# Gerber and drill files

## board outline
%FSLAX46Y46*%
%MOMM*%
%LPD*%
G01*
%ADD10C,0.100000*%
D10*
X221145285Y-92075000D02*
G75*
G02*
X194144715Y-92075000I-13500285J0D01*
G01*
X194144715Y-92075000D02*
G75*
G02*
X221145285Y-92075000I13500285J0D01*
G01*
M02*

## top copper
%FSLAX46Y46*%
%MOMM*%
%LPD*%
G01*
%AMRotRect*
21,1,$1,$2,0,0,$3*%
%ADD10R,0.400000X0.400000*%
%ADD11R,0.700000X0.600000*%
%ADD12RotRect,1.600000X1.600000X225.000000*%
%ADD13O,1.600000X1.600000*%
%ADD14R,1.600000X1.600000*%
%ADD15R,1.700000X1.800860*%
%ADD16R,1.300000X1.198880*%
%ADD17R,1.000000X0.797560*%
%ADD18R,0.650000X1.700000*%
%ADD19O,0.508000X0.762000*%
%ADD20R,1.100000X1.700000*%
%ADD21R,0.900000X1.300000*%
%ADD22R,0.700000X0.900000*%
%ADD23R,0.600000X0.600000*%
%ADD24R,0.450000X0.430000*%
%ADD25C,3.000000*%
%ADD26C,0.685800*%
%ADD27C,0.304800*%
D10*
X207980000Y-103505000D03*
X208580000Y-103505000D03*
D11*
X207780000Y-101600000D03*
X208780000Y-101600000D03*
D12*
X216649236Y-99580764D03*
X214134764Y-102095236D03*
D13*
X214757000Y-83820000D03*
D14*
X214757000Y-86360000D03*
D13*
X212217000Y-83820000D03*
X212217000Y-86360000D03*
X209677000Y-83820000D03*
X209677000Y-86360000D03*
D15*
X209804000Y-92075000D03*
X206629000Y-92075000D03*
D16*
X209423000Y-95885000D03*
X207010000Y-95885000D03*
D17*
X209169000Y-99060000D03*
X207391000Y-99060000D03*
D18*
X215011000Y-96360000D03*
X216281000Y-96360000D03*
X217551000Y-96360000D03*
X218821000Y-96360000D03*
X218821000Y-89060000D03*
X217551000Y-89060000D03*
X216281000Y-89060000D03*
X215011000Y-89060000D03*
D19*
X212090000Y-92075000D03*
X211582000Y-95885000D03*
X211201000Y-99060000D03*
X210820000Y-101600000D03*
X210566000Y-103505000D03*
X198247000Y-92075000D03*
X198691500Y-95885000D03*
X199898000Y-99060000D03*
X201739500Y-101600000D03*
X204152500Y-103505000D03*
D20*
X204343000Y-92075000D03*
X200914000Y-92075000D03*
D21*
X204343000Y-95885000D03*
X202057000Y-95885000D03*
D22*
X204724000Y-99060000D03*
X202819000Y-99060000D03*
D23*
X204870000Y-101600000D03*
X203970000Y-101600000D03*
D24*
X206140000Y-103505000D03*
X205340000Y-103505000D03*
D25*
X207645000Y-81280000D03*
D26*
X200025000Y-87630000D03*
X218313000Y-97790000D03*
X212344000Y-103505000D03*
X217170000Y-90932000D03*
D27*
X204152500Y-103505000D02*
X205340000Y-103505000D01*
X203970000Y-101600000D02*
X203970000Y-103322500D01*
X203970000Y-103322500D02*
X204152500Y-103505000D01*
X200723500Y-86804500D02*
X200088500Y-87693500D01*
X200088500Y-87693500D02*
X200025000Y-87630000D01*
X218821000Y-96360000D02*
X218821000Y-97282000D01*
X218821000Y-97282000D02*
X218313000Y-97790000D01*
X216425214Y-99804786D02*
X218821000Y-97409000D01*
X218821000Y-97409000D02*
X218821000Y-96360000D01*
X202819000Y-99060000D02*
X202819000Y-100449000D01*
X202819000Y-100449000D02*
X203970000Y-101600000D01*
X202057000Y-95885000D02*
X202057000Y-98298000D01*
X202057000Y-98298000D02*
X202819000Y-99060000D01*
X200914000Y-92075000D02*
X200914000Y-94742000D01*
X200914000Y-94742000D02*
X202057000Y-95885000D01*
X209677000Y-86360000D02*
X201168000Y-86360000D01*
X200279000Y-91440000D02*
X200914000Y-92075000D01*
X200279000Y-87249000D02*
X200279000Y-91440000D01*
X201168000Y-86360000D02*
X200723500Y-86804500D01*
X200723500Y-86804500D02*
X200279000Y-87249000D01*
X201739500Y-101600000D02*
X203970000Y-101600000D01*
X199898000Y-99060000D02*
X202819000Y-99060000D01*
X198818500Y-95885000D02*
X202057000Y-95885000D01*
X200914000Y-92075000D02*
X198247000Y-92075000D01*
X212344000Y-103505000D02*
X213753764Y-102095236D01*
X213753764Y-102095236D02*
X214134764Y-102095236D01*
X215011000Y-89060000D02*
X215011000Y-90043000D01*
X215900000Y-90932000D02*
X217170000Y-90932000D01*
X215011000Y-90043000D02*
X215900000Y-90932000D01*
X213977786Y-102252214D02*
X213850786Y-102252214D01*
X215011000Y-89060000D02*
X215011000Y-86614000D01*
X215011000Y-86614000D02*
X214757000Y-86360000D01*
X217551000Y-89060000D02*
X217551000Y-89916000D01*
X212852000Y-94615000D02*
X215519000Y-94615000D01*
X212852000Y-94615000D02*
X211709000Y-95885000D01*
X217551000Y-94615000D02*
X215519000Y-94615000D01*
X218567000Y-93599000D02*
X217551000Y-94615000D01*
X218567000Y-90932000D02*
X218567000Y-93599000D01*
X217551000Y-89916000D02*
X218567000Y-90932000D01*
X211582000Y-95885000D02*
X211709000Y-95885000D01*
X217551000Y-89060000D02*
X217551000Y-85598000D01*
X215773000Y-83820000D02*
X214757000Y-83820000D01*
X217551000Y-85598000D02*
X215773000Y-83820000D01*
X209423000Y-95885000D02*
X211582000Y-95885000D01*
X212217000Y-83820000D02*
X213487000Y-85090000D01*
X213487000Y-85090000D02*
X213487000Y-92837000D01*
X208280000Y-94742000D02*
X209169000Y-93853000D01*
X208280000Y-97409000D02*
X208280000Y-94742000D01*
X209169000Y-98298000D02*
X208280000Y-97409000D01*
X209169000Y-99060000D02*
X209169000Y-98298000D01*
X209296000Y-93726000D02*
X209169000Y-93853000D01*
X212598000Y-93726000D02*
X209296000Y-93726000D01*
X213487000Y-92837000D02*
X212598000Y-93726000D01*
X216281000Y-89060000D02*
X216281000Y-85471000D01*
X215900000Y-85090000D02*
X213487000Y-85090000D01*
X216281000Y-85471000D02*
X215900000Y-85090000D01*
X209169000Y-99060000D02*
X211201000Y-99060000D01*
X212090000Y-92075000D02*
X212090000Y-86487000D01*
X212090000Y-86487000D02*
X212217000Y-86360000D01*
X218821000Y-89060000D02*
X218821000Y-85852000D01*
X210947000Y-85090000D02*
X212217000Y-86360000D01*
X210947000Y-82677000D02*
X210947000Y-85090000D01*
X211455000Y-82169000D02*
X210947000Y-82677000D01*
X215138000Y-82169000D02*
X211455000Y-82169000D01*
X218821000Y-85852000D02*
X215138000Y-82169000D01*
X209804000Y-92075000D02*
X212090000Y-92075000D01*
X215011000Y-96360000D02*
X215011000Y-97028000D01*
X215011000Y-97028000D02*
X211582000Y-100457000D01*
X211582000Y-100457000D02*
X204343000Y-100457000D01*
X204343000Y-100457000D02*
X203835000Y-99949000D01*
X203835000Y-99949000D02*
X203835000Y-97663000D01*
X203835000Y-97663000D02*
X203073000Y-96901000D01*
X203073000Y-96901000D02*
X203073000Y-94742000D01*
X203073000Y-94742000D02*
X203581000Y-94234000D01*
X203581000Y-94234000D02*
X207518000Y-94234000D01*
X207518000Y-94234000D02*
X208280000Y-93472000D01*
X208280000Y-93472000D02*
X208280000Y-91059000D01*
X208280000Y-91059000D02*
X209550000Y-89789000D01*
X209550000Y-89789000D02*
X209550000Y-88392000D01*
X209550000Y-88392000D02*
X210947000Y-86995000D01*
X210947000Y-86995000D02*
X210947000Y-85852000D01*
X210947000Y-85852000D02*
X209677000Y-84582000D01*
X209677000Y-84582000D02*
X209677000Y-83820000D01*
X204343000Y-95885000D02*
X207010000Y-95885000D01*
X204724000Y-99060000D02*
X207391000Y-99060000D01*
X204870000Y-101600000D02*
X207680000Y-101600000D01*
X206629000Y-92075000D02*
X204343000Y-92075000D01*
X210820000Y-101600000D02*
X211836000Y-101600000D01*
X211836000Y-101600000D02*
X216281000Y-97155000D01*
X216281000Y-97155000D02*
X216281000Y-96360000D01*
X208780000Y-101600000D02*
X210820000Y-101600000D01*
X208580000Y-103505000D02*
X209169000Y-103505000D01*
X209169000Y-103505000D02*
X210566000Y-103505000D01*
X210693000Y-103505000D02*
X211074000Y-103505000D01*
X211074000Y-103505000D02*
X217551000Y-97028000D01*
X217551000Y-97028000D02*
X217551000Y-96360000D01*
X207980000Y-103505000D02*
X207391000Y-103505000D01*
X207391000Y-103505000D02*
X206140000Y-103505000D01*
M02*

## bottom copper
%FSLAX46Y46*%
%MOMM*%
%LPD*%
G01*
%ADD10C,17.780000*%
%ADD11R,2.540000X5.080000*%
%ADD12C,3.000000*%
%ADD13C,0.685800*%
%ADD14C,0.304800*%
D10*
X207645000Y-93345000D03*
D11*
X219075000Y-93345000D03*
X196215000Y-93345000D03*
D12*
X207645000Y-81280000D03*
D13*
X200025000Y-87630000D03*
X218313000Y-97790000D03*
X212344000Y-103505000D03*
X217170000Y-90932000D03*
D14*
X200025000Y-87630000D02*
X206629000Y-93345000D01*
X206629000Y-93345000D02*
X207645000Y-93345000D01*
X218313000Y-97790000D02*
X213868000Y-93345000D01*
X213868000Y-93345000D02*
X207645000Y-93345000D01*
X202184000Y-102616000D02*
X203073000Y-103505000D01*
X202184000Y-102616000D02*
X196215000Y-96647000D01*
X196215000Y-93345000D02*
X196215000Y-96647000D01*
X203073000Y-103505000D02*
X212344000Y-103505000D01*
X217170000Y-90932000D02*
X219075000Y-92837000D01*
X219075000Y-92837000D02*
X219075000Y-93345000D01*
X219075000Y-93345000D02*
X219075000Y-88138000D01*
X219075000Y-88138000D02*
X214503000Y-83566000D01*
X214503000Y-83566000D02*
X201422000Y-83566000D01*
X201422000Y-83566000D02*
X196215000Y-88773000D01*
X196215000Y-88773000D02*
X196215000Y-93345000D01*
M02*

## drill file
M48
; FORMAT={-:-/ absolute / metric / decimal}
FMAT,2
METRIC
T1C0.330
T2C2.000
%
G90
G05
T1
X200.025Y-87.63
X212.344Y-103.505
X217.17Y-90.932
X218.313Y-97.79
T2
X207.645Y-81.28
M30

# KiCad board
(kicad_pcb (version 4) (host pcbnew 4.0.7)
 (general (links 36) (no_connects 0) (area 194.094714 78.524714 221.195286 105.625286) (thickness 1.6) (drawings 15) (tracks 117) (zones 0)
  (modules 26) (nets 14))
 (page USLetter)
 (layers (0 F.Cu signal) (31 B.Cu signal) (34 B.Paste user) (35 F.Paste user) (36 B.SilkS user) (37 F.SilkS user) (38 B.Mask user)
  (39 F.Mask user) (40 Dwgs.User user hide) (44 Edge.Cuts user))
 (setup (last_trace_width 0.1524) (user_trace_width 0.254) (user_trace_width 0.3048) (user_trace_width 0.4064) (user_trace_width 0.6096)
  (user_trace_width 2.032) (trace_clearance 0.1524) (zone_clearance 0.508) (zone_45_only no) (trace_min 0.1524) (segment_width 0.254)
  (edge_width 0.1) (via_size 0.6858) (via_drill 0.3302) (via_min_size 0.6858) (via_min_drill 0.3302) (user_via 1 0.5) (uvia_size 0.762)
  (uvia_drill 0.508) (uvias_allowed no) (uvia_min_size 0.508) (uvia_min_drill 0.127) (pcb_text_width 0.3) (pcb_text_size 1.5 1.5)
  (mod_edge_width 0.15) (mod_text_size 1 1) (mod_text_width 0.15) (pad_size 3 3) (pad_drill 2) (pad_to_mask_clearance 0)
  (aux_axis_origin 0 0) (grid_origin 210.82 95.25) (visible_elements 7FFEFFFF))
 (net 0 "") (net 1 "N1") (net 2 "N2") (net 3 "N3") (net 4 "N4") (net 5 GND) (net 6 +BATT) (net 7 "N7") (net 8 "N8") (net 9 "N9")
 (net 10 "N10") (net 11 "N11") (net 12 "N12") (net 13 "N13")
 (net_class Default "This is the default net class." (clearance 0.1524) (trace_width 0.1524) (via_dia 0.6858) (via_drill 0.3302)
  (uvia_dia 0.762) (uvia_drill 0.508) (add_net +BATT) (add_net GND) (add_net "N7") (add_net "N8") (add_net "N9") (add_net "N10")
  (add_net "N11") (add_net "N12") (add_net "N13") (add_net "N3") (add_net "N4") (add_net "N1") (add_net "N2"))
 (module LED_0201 (layer F.Cu) (at 208.28 103.505)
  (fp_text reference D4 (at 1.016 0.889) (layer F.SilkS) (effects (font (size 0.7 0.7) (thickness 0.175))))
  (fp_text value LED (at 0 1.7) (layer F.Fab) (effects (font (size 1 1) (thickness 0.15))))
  (pad 1 smd rect (at -0.3 0) (size 0.4 0.4) (layers F.Cu F.Paste F.Mask) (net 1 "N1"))
  (pad 2 smd rect (at 0.3 0) (size 0.4 0.4) (layers F.Cu F.Paste F.Mask) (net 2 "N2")))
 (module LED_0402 (layer F.Cu) (at 208.28 101.6)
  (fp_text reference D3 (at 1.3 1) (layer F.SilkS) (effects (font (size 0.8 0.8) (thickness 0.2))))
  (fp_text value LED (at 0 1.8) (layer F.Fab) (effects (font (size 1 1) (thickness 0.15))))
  (pad 1 smd rect (at -0.5 0) (size 0.7 0.6) (layers F.Cu F.Paste F.Mask) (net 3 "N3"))
  (pad 2 smd rect (at 0.5 0) (size 0.7 0.6) (layers F.Cu F.Paste F.Mask) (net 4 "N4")))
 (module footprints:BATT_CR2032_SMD (layer B.Cu) (at 207.645 93.345 180)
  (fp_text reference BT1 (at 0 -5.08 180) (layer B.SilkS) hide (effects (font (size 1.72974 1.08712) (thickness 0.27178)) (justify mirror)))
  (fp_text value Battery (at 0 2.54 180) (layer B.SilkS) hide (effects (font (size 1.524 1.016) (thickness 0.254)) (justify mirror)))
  (pad 2 smd circle (at 0 0 180) (size 17.78 17.78) (layers B.Cu B.Paste B.Mask) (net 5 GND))
  (pad 1 smd rect (at -11.43 0 180) (size 2.54 5.08) (layers B.Cu B.Paste B.Mask) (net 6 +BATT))
  (pad 1 smd rect (at 11.43 0 180) (size 2.54 5.08) (layers B.Cu B.Paste B.Mask) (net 6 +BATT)))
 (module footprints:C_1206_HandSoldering (layer F.Cu) (at 215.392 100.838 225)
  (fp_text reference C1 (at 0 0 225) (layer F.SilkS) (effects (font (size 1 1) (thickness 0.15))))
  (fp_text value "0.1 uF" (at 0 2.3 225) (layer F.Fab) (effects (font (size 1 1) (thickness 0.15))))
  (pad 1 smd rect (at -1.778 0 225) (size 1.6 1.6) (layers F.Cu F.Paste F.Mask) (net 5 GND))
  (pad 2 smd rect (at 1.778 0 225) (size 1.6 1.6) (layers F.Cu F.Paste F.Mask) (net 6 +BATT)))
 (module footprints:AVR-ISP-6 (layer F.Cu) (at 214.757 83.82 270)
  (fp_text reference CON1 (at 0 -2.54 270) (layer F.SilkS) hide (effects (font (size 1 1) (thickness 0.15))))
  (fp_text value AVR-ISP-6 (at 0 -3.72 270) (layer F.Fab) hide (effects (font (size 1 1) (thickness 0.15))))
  (pad 1 smd oval (at 0 0 270) (size 1.6 1.6) (layers F.Cu F.Paste F.Mask) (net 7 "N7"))
  (pad 2 smd rect (at 2.54 0 270) (size 1.6 1.6) (layers F.Cu F.Paste F.Mask) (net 6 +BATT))
  (pad 3 smd oval (at 0 2.54 270) (size 1.6 1.6) (layers F.Cu F.Paste F.Mask) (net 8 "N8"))
  (pad 4 smd oval (at 2.54 2.54 270) (size 1.6 1.6) (layers F.Cu F.Paste F.Mask) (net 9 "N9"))
  (pad 5 smd oval (at 0 5.08 270) (size 1.6 1.6) (layers F.Cu F.Paste F.Mask) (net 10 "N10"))
  (pad 6 smd oval (at 2.54 5.08 270) (size 1.6 1.6) (layers F.Cu F.Paste F.Mask) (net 5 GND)))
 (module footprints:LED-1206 (layer F.Cu) (at 208.28 92.075)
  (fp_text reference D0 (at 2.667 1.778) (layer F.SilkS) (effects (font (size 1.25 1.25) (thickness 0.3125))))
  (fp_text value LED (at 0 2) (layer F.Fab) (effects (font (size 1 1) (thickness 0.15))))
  (pad 2 smd rect (at 1.524 0 180) (size 1.7 1.80086) (layers F.Cu F.Paste F.Mask) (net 9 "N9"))
  (pad 1 smd rect (at -1.651 0 180) (size 1.7 1.80086) (layers F.Cu F.Paste F.Mask) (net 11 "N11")))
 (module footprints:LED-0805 (layer F.Cu) (at 208.28 95.885)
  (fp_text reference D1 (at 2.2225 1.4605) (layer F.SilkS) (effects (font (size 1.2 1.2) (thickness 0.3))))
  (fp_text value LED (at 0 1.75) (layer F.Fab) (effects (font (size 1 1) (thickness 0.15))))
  (pad 2 smd rect (at 1.143 0 180) (size 1.3 1.19888) (layers F.Cu F.Paste F.Mask) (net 7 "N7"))
  (pad 1 smd rect (at -1.27 0 180) (size 1.3 1.19888) (layers F.Cu F.Paste F.Mask) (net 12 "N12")))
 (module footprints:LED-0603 (layer F.Cu) (at 208.28 99.06)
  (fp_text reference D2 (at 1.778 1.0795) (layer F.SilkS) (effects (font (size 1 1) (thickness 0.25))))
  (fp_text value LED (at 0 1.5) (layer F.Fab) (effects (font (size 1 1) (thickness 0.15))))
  (pad 2 smd rect (at 0.889 0 180) (size 1 0.79756) (layers F.Cu F.Paste F.Mask) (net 8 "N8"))
  (pad 1 smd rect (at -0.889 0 180) (size 1 0.79756) (layers F.Cu F.Paste F.Mask) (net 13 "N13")))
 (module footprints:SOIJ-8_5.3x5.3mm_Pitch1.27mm (layer F.Cu) (at 216.916 92.71 90)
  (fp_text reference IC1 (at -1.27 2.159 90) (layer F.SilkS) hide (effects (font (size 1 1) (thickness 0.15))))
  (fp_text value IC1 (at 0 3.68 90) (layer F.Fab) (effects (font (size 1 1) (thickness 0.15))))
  (pad 1 smd rect (at -3.65 -1.905 90) (size 1.7 0.65) (layers F.Cu F.Paste F.Mask) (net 10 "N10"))
  (pad 2 smd rect (at -3.65 -0.635 90) (size 1.7 0.65) (layers F.Cu F.Paste F.Mask) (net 4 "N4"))
  (pad 3 smd rect (at -3.65 0.635 90) (size 1.7 0.65) (layers F.Cu F.Paste F.Mask) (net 2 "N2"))
  (pad 4 smd rect (at -3.65 1.905 90) (size 1.7 0.65) (layers F.Cu F.Paste F.Mask) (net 5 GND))
  (pad 5 smd rect (at 3.65 1.905 90) (size 1.7 0.65) (layers F.Cu F.Paste F.Mask) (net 9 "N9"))
  (pad 6 smd rect (at 3.65 0.635 90) (size 1.7 0.65) (layers F.Cu F.Paste F.Mask) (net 7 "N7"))
  (pad 7 smd rect (at 3.65 -0.635 90) (size 1.7 0.65) (layers F.Cu F.Paste F.Mask) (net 8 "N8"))
  (pad 8 smd rect (at 3.65 -1.905 90) (size 1.7 0.65) (layers F.Cu F.Paste F.Mask) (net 6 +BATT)))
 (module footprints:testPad (layer F.Cu) (at 212.09 92.075)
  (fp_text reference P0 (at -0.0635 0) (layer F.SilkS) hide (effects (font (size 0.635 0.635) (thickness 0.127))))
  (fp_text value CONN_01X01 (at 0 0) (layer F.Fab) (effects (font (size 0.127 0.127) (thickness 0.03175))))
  (pad 1 smd oval (at 0 0) (size 0.508 0.762) (layers F.Cu F.Paste F.Mask) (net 9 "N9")))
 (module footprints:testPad (layer F.Cu) (at 211.582 95.885)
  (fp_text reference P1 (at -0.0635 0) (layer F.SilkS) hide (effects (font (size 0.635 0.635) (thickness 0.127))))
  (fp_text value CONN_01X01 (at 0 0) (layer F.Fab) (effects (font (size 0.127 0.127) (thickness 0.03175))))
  (pad 1 smd oval (at 0 0) (size 0.508 0.762) (layers F.Cu F.Paste F.Mask) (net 7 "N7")))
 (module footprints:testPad (layer F.Cu) (at 211.201 99.06)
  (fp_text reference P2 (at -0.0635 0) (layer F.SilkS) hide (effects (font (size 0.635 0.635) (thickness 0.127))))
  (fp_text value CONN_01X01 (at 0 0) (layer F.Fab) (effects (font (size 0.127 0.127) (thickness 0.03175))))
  (pad 1 smd oval (at 0 0) (size 0.508 0.762) (layers F.Cu F.Paste F.Mask) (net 8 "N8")))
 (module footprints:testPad (layer F.Cu) (at 210.82 101.6)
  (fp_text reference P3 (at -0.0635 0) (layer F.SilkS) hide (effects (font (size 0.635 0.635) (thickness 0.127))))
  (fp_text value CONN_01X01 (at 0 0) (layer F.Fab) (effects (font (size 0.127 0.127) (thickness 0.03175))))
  (pad 1 smd oval (at 0 0) (size 0.508 0.762) (layers F.Cu F.Paste F.Mask) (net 4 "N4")))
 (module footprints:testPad (layer F.Cu) (at 210.566 103.505)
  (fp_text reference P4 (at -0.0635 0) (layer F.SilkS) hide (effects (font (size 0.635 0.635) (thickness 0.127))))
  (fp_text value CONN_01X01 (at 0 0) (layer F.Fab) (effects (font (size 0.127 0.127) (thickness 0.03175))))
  (pad 1 smd oval (at 0 0) (size 0.508 0.762) (layers F.Cu F.Paste F.Mask) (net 2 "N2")))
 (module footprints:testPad (layer F.Cu) (at 198.247 92.075)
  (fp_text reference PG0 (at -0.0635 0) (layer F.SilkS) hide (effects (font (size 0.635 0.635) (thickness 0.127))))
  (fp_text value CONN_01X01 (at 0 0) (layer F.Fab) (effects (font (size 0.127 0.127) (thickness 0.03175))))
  (pad 1 smd oval (at 0 0) (size 0.508 0.762) (layers F.Cu F.Paste F.Mask) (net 5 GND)))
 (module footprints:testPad (layer F.Cu) (at 198.6915 95.885)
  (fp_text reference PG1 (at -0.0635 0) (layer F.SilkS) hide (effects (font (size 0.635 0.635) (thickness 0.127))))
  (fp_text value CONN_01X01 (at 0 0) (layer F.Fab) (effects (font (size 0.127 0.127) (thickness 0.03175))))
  (pad 1 smd oval (at 0 0) (size 0.508 0.762) (layers F.Cu F.Paste F.Mask) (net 5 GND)))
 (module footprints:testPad (layer F.Cu) (at 199.898 99.06)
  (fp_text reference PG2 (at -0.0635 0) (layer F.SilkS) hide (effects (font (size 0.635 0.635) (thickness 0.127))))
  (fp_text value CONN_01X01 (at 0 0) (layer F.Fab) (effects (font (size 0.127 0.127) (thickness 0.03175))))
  (pad 1 smd oval (at 0 0) (size 0.508 0.762) (layers F.Cu F.Paste F.Mask) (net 5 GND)))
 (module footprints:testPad (layer F.Cu) (at 201.7395 101.6)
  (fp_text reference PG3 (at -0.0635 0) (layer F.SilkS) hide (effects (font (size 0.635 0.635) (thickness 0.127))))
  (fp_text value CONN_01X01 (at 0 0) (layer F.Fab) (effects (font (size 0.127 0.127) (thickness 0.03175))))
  (pad 1 smd oval (at 0 0) (size 0.508 0.762) (layers F.Cu F.Paste F.Mask) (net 5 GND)))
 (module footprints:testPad (layer F.Cu) (at 204.1525 103.505)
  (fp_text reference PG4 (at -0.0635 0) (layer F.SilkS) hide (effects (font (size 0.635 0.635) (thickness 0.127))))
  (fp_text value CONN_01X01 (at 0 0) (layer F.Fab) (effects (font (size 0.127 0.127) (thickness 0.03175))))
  (pad 1 smd oval (at 0 0) (size 0.508 0.762) (layers F.Cu F.Paste F.Mask) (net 5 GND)))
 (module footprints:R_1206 (layer F.Cu) (at 202.565 92.075 180)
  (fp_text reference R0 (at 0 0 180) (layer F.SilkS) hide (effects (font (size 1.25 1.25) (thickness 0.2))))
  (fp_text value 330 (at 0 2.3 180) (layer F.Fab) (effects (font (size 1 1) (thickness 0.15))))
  (pad 1 smd rect (at -1.778 0 180) (size 1.1 1.7) (layers F.Cu F.Paste F.Mask) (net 11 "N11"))
  (pad 2 smd rect (at 1.651 0 180) (size 1.1 1.7) (layers F.Cu F.Paste F.Mask) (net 5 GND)))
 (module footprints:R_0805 (layer F.Cu) (at 203.2 95.885 180)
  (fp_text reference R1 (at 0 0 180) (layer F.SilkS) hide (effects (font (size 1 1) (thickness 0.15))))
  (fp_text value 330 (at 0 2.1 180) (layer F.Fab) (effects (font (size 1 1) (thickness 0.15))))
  (pad 1 smd rect (at -1.143 0 180) (size 0.9 1.3) (layers F.Cu F.Paste F.Mask) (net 12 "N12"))
  (pad 2 smd rect (at 1.143 0 180) (size 0.9 1.3) (layers F.Cu F.Paste F.Mask) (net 5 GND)))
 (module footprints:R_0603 (layer F.Cu) (at 203.835 99.06 180)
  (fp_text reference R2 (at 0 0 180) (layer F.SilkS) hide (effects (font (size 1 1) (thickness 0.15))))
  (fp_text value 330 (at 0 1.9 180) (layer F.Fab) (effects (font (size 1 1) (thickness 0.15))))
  (pad 1 smd rect (at -0.889 0 180) (size 0.7 0.9) (layers F.Cu F.Paste F.Mask) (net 13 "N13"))
  (pad 2 smd rect (at 1.016 0 180) (size 0.7 0.9) (layers F.Cu F.Paste F.Mask) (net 5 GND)))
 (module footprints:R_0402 (layer F.Cu) (at 204.47 101.6 180)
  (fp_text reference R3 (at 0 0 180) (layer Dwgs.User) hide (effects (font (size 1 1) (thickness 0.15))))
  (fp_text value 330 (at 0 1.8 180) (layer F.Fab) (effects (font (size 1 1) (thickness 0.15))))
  (pad 1 smd rect (at -0.4 0 180) (size 0.6 0.6) (layers F.Cu F.Paste F.Mask) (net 3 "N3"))
  (pad 2 smd rect (at 0.5 0 180) (size 0.6 0.6) (layers F.Cu F.Paste F.Mask) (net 5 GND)))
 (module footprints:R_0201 (layer F.Cu) (at 205.74 103.505 180)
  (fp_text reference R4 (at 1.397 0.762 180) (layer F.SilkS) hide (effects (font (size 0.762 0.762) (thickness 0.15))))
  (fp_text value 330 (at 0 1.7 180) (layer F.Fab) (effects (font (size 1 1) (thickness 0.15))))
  (pad 1 smd rect (at -0.4 0 180) (size 0.45 0.43) (layers F.Cu F.Paste F.Mask) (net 1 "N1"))
  (pad 2 smd rect (at 0.4 0 180) (size 0.45 0.43) (layers F.Cu F.Paste F.Mask) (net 5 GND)))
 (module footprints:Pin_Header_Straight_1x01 (layer F.Cu) (at 207.645 81.28)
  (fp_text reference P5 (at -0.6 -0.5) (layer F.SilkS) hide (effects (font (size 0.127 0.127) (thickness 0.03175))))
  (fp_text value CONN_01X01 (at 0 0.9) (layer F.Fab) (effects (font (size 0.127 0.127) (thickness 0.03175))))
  (pad 1 thru_hole circle (at 0 0) (size 3 3) (drill 2) (layers *.Cu *.Mask)))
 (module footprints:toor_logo (layer F.Cu) (at 202.565 85.725)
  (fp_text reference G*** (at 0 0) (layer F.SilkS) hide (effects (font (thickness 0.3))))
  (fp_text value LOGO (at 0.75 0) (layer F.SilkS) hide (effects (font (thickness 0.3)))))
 (gr_circle (center 207.645 92.075) (end 197.485 83.185) (layer Edge.Cuts) (width 0.1))
 (segment (start 204.1525 103.505) (end 205.34 103.505) (width 0.3048) (layer F.Cu) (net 5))
 (segment (start 203.97 101.6) (end 203.97 103.3225) (width 0.3048) (layer F.Cu) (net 5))
 (segment (start 203.97 103.3225) (end 204.1525 103.505) (width 0.3048) (layer F.Cu) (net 5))
 (segment (start 200.7235 86.8045) (end 200.0885 87.6935) (width 0.3048) (layer F.Cu) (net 5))
 (segment (start 200.025 87.63) (end 206.629 93.345) (width 0.3048) (layer B.Cu) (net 5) (status 20))
 (via (at 200.025 87.63) (size 0.6858) (drill 0.3302) (layers F.Cu B.Cu) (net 5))
 (segment (start 200.0885 87.6935) (end 200.025 87.63) (width 0.3048) (layer F.Cu) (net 5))
 (segment (start 206.629 93.345) (end 207.645 93.345) (width 0.3048) (layer B.Cu) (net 5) (status 30))
 (segment (start 218.821 96.36) (end 218.821 97.282) (width 0.3048) (layer F.Cu) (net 5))
 (segment (start 218.313 97.79) (end 213.868 93.345) (width 0.3048) (layer B.Cu) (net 5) (status 20))
 (via (at 218.313 97.79) (size 0.6858) (drill 0.3302) (layers F.Cu B.Cu) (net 5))
 (segment (start 218.821 97.282) (end 218.313 97.79) (width 0.3048) (layer F.Cu) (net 5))
 (segment (start 213.868 93.345) (end 207.645 93.345) (width 0.3048) (layer B.Cu) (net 5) (status 30))
 (segment (start 216.425214 99.804786) (end 218.821 97.409) (width 0.3048) (layer F.Cu) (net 5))
 (segment (start 218.821 97.409) (end 218.821 96.36) (width 0.3048) (layer F.Cu) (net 5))
 (segment (start 202.819 99.06) (end 202.819 100.449) (width 0.3048) (layer F.Cu) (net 5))
 (segment (start 202.819 100.449) (end 203.97 101.6) (width 0.3048) (layer F.Cu) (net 5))
 (segment (start 202.057 95.885) (end 202.057 98.298) (width 0.3048) (layer F.Cu) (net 5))
 (segment (start 202.057 98.298) (end 202.819 99.06) (width 0.3048) (layer F.Cu) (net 5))
 (segment (start 200.914 92.075) (end 200.914 94.742) (width 0.3048) (layer F.Cu) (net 5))
 (segment (start 200.914 94.742) (end 202.057 95.885) (width 0.3048) (layer F.Cu) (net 5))
 (segment (start 209.677 86.36) (end 201.168 86.36) (width 0.3048) (layer F.Cu) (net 5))
 (segment (start 200.279 91.44) (end 200.914 92.075) (width 0.3048) (layer F.Cu) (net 5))
 (segment (start 200.279 87.249) (end 200.279 91.44) (width 0.3048) (layer F.Cu) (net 5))
 (segment (start 201.168 86.36) (end 200.7235 86.8045) (width 0.3048) (layer F.Cu) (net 5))
 (segment (start 200.7235 86.8045) (end 200.279 87.249) (width 0.3048) (layer F.Cu) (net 5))
 (segment (start 201.7395 101.6) (end 203.97 101.6) (width 0.3048) (layer F.Cu) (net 5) (status 10))
 (segment (start 199.898 99.06) (end 202.819 99.06) (width 0.3048) (layer F.Cu) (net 5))
 (segment (start 198.8185 95.885) (end 202.057 95.885) (width 0.3048) (layer F.Cu) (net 5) (status 10))
 (segment (start 200.914 92.075) (end 198.247 92.075) (width 0.3048) (layer F.Cu) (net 5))
 (segment (start 202.184 102.616) (end 203.073 103.505) (width 0.3048) (layer B.Cu) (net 6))
 (segment (start 202.184 102.616) (end 196.215 96.647) (width 0.3048) (layer B.Cu) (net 6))
 (segment (start 196.215 93.345) (end 196.215 96.647) (width 0.3048) (layer B.Cu) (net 6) (status 10))
 (segment (start 212.344 103.505) (end 213.753764 102.095236) (width 0.3048) (layer F.Cu) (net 6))
 (via (at 212.344 103.505) (size 0.6858) (drill 0.3302) (layers F.Cu B.Cu) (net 6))
 (segment (start 203.073 103.505) (end 212.344 103.505) (width 0.3048) (layer B.Cu) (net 6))
 (segment (start 213.753764 102.095236) (end 214.134764 102.095236) (width 0.3048) (layer F.Cu) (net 6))
 (segment (start 215.011 89.06) (end 215.011 90.043) (width 0.3048) (layer F.Cu) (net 6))
 (segment (start 217.17 90.932) (end 219.075 92.837) (width 0.3048) (layer B.Cu) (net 6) (status 20))
 (via (at 217.17 90.932) (size 0.6858) (drill 0.3302) (layers F.Cu B.Cu) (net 6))
 (segment (start 215.9 90.932) (end 217.17 90.932) (width 0.3048) (layer F.Cu) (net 6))
 (segment (start 215.011 90.043) (end 215.9 90.932) (width 0.3048) (layer F.Cu) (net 6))
 (segment (start 219.075 92.837) (end 219.075 93.345) (width 0.3048) (layer B.Cu) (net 6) (status 30))
 (segment (start 219.075 93.345) (end 219.075 88.138) (width 0.3048) (layer B.Cu) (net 6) (status 10))
 (segment (start 219.075 88.138) (end 214.503 83.566) (width 0.3048) (layer B.Cu) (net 6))
 (segment (start 214.503 83.566) (end 201.422 83.566) (width 0.3048) (layer B.Cu) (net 6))
 (segment (start 201.422 83.566) (end 196.215 88.773) (width 0.3048) (layer B.Cu) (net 6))
 (segment (start 196.215 88.773) (end 196.215 93.345) (width 0.3048) (layer B.Cu) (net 6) (status 20))
 (segment (start 213.977786 102.252214) (end 213.850786 102.252214) (width 0.3048) (layer F.Cu) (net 6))
 (segment (start 215.011 89.06) (end 215.011 86.614) (width 0.3048) (layer F.Cu) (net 6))
 (segment (start 215.011 86.614) (end 214.757 86.36) (width 0.3048) (layer F.Cu) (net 6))
 (segment (start 217.551 89.06) (end 217.551 89.916) (width 0.3048) (layer F.Cu) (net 7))
 (segment (start 212.852 94.615) (end 215.519 94.615) (width 0.3048) (layer F.Cu) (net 7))
 (segment (start 212.852 94.615) (end 211.709 95.885) (width 0.3048) (layer F.Cu) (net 7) (status 20))
 (segment (start 217.551 94.615) (end 215.519 94.615) (width 0.3048) (layer F.Cu) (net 7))
 (segment (start 218.567 93.599) (end 217.551 94.615) (width 0.3048) (layer F.Cu) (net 7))
 (segment (start 218.567 90.932) (end 218.567 93.599) (width 0.3048) (layer F.Cu) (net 7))
 (segment (start 217.551 89.916) (end 218.567 90.932) (width 0.3048) (layer F.Cu) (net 7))
 (segment (start 211.582 95.885) (end 211.709 95.885) (width 0.3048) (layer F.Cu) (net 7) (status 30))
 (segment (start 217.551 89.06) (end 217.551 85.598) (width 0.3048) (layer F.Cu) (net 7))
 (segment (start 215.773 83.82) (end 214.757 83.82) (width 0.3048) (layer F.Cu) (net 7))
 (segment (start 217.551 85.598) (end 215.773 83.82) (width 0.3048) (layer F.Cu) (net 7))
 (segment (start 209.423 95.885) (end 211.582 95.885) (width 0.3048) (layer F.Cu) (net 7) (status 20))
 (segment (start 212.217 83.82) (end 213.487 85.09) (width 0.3048) (layer F.Cu) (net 8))
 (segment (start 213.487 85.09) (end 213.487 92.837) (width 0.3048) (layer F.Cu) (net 8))
 (segment (start 208.28 94.742) (end 209.169 93.853) (width 0.3048) (layer F.Cu) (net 8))
 (segment (start 208.28 97.409) (end 208.28 94.742) (width 0.3048) (layer F.Cu) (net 8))
 (segment (start 209.169 98.298) (end 208.28 97.409) (width 0.3048) (layer F.Cu) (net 8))
 (segment (start 209.169 99.06) (end 209.169 98.298) (width 0.3048) (layer F.Cu) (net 8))
 (segment (start 209.296 93.726) (end 209.169 93.853) (width 0.3048) (layer F.Cu) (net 8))
 (segment (start 212.598 93.726) (end 209.296 93.726) (width 0.3048) (layer F.Cu) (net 8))
 (segment (start 213.487 92.837) (end 212.598 93.726) (width 0.3048) (layer F.Cu) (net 8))
 (segment (start 216.281 89.06) (end 216.281 85.471) (width 0.3048) (layer F.Cu) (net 8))
 (segment (start 215.9 85.09) (end 213.487 85.09) (width 0.3048) (layer F.Cu) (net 8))
 (segment (start 216.281 85.471) (end 215.9 85.09) (width 0.3048) (layer F.Cu) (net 8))
 (segment (start 209.169 99.06) (end 211.201 99.06) (width 0.3048) (layer F.Cu) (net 8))
 (segment (start 212.09 92.075) (end 212.09 86.487) (width 0.3048) (layer F.Cu) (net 9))
 (segment (start 212.09 86.487) (end 212.217 86.36) (width 0.3048) (layer F.Cu) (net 9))
 (segment (start 218.821 89.06) (end 218.821 85.852) (width 0.3048) (layer F.Cu) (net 9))
 (segment (start 210.947 85.09) (end 212.217 86.36) (width 0.3048) (layer F.Cu) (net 9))
 (segment (start 210.947 82.677) (end 210.947 85.09) (width 0.3048) (layer F.Cu) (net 9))
 (segment (start 211.455 82.169) (end 210.947 82.677) (width 0.3048) (layer F.Cu) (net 9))
 (segment (start 215.138 82.169) (end 211.455 82.169) (width 0.3048) (layer F.Cu) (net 9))
 (segment (start 218.821 85.852) (end 215.138 82.169) (width 0.3048) (layer F.Cu) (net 9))
 (segment (start 209.804 92.075) (end 212.09 92.075) (width 0.3048) (layer F.Cu) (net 9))
 (segment (start 215.011 96.36) (end 215.011 97.028) (width 0.3048) (layer F.Cu) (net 10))
 (segment (start 215.011 97.028) (end 211.582 100.457) (width 0.3048) (layer F.Cu) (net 10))
 (segment (start 211.582 100.457) (end 204.343 100.457) (width 0.3048) (layer F.Cu) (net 10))
 (segment (start 204.343 100.457) (end 203.835 99.949) (width 0.3048) (layer F.Cu) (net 10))
 (segment (start 203.835 99.949) (end 203.835 97.663) (width 0.3048) (layer F.Cu) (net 10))
 (segment (start 203.835 97.663) (end 203.073 96.901) (width 0.3048) (layer F.Cu) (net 10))
 (segment (start 203.073 96.901) (end 203.073 94.742) (width 0.3048) (layer F.Cu) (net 10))
 (segment (start 203.073 94.742) (end 203.581 94.234) (width 0.3048) (layer F.Cu) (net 10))
 (segment (start 203.581 94.234) (end 207.518 94.234) (width 0.3048) (layer F.Cu) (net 10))
 (segment (start 207.518 94.234) (end 208.28 93.472) (width 0.3048) (layer F.Cu) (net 10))
 (segment (start 208.28 93.472) (end 208.28 91.059) (width 0.3048) (layer F.Cu) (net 10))
 (segment (start 208.28 91.059) (end 209.55 89.789) (width 0.3048) (layer F.Cu) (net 10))
 (segment (start 209.55 89.789) (end 209.55 88.392) (width 0.3048) (layer F.Cu) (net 10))
 (segment (start 209.55 88.392) (end 210.947 86.995) (width 0.3048) (layer F.Cu) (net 10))
 (segment (start 210.947 86.995) (end 210.947 85.852) (width 0.3048) (layer F.Cu) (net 10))
 (segment (start 210.947 85.852) (end 209.677 84.582) (width 0.3048) (layer F.Cu) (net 10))
 (segment (start 209.677 84.582) (end 209.677 83.82) (width 0.3048) (layer F.Cu) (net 10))
 (segment (start 204.343 95.885) (end 207.01 95.885) (width 0.3048) (layer F.Cu) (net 12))
 (segment (start 204.724 99.06) (end 207.391 99.06) (width 0.3048) (layer F.Cu) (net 13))
 (segment (start 204.87 101.6) (end 207.68 101.6) (width 0.3048) (layer F.Cu) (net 3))
 (segment (start 206.629 92.075) (end 204.343 92.075) (width 0.3048) (layer F.Cu) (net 11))
 (segment (start 210.82 101.6) (end 211.836 101.6) (width 0.3048) (layer F.Cu) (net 4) (status 10))
 (segment (start 211.836 101.6) (end 216.281 97.155) (width 0.3048) (layer F.Cu) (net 4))
 (segment (start 216.281 97.155) (end 216.281 96.36) (width 0.3048) (layer F.Cu) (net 4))
 (segment (start 208.78 101.6) (end 210.82 101.6) (width 0.3048) (layer F.Cu) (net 4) (status 20))
 (segment (start 208.58 103.505) (end 209.169 103.505) (width 0.3048) (layer F.Cu) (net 2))
 (segment (start 209.169 103.505) (end 210.566 103.505) (width 0.3048) (layer F.Cu) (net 2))
 (segment (start 210.693 103.505) (end 211.074 103.505) (width 0.3048) (layer F.Cu) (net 2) (status 10))
 (segment (start 211.074 103.505) (end 217.551 97.028) (width 0.3048) (layer F.Cu) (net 2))
 (segment (start 217.551 97.028) (end 217.551 96.36) (width 0.3048) (layer F.Cu) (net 2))
 (segment (start 207.98 103.505) (end 207.391 103.505) (width 0.3048) (layer F.Cu) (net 1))
 (segment (start 207.391 103.505) (end 206.14 103.505) (width 0.3048) (layer F.Cu) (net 1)))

